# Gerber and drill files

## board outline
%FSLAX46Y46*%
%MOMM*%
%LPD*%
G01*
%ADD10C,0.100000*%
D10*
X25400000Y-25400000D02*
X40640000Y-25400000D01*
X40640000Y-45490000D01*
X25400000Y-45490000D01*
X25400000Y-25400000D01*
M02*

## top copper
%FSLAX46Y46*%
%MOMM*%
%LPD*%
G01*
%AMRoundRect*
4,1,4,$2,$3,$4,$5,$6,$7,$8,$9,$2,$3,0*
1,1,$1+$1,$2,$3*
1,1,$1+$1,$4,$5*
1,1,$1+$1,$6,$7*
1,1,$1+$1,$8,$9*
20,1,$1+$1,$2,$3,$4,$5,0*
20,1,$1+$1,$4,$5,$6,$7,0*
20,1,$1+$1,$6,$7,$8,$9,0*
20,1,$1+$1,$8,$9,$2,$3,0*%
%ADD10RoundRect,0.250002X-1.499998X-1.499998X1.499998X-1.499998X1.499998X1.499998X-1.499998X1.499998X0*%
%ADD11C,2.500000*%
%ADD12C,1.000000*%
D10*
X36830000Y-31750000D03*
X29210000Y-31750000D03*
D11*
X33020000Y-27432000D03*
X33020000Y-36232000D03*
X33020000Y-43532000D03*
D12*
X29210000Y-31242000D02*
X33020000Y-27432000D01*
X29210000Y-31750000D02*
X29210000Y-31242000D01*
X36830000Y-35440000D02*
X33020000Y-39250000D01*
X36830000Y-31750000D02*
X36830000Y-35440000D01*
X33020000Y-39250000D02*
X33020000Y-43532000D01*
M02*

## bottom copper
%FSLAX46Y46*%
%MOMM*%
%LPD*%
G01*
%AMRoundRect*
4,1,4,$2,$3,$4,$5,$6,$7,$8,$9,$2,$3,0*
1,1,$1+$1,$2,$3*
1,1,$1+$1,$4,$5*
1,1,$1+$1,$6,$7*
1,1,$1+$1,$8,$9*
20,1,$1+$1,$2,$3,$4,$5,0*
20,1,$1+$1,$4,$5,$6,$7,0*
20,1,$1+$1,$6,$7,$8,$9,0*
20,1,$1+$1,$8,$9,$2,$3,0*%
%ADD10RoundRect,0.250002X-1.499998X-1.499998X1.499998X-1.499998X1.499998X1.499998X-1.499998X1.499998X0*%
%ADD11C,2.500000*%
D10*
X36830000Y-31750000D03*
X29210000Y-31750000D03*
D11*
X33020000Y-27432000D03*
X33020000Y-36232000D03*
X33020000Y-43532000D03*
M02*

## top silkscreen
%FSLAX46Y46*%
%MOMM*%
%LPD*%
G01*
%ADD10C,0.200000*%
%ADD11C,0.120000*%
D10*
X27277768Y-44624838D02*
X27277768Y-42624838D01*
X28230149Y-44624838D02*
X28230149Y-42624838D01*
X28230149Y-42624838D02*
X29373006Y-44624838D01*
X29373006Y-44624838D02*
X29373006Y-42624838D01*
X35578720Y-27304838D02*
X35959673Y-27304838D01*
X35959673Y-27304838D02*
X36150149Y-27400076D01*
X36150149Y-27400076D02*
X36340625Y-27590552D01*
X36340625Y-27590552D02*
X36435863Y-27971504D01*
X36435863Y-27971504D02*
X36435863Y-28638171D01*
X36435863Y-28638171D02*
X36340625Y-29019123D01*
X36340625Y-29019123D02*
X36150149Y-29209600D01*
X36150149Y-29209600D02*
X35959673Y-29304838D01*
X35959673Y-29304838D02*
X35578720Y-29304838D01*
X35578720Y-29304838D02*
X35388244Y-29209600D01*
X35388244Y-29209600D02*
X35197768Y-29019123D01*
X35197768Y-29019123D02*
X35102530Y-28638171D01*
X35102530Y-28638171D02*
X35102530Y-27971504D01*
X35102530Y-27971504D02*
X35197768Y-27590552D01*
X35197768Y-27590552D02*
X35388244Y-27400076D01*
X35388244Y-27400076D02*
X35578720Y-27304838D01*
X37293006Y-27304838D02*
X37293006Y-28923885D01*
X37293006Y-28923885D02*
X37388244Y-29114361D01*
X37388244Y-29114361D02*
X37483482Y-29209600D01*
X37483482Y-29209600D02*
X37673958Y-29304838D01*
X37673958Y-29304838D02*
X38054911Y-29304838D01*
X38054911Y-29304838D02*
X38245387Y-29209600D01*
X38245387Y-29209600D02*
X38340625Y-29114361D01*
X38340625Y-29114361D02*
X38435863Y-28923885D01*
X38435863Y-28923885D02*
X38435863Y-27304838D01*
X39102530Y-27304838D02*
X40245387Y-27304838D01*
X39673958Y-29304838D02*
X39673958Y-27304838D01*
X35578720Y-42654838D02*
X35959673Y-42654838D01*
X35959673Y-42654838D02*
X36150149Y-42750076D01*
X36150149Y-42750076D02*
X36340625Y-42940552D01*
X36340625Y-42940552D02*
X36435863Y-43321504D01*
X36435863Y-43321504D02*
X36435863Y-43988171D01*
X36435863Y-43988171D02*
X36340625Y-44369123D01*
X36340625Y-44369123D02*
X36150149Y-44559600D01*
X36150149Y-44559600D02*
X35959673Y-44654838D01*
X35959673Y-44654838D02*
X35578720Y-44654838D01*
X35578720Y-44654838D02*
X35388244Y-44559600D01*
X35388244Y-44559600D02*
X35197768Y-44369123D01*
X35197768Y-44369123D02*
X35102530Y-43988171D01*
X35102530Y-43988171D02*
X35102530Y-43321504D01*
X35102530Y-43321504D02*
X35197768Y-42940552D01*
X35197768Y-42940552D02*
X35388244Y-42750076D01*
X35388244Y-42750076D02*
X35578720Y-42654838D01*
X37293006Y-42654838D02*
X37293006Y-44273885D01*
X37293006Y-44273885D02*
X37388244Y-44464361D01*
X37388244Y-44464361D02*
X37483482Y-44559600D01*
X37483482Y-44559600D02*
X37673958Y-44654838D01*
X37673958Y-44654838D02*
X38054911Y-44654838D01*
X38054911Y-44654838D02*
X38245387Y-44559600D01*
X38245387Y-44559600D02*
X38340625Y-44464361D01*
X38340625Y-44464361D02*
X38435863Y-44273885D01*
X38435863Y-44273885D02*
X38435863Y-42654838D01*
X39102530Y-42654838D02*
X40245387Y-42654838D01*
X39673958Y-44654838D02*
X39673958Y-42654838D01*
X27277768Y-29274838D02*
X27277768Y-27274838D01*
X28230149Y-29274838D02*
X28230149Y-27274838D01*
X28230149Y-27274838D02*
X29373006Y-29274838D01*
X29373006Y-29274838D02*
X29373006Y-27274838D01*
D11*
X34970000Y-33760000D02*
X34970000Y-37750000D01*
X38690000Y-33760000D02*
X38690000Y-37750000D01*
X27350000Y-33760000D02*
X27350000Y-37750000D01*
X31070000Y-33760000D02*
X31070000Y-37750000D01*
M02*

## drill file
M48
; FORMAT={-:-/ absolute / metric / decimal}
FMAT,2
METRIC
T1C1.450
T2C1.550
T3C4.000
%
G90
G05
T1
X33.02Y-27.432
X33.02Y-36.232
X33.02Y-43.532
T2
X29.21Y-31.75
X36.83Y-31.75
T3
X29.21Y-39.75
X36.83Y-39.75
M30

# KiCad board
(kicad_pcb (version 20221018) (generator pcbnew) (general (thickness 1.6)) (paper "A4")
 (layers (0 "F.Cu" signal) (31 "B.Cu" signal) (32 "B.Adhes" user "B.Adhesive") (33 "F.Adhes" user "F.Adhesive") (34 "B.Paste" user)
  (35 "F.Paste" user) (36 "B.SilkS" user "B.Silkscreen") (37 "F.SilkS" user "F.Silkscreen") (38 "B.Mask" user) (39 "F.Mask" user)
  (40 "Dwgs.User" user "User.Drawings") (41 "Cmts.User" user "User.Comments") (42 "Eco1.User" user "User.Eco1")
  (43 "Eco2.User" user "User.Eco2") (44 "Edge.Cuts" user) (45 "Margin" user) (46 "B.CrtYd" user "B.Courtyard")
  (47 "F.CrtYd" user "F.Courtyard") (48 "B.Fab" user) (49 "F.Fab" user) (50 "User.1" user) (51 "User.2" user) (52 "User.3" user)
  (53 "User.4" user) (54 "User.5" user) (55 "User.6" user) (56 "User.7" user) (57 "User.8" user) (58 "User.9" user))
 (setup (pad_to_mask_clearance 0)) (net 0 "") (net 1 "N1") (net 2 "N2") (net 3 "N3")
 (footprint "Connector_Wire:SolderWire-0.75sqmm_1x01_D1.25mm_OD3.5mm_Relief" (layer "F.Cu") (at 36.83 31.75)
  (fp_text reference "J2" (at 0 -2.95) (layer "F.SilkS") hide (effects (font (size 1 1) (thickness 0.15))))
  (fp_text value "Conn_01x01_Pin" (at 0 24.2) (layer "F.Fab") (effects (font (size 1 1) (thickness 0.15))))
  (fp_line (start -1.86 2.01) (end -1.86 6) (stroke (width 0.12) (type solid)) (layer "F.SilkS"))
  (fp_line (start 1.86 2.01) (end 1.86 6) (stroke (width 0.12) (type solid)) (layer "F.SilkS"))
  (pad "" np_thru_hole circle (at 0 8) (size 4 4) (drill 4) (layers "*.Cu" "*.Mask"))
  (pad "1" thru_hole roundrect (at 0 0) (size 3.5 3.5) (drill 1.55) (layers "*.Cu" "*.Mask") (roundrect_rratio 0.071429) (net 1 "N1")))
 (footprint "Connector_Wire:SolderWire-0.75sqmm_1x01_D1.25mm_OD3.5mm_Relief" (layer "F.Cu") (at 29.21 31.75)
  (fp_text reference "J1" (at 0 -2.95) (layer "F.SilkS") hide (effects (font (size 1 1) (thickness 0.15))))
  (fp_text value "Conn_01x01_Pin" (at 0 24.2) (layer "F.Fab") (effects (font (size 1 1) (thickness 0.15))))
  (fp_line (start -1.86 2.01) (end -1.86 6) (stroke (width 0.12) (type solid)) (layer "F.SilkS"))
  (fp_line (start 1.86 2.01) (end 1.86 6) (stroke (width 0.12) (type solid)) (layer "F.SilkS"))
  (pad "" np_thru_hole circle (at 0 8) (size 4 4) (drill 4) (layers "*.Cu" "*.Mask"))
  (pad "1" thru_hole roundrect (at 0 0) (size 3.5 3.5) (drill 1.55) (layers "*.Cu" "*.Mask") (roundrect_rratio 0.071429) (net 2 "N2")))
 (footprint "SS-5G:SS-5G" (layer "F.Cu") (at 33.02 27.432)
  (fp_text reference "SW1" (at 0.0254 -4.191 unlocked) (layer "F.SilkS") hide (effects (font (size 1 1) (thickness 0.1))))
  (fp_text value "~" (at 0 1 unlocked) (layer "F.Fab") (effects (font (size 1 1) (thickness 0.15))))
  (pad "1" thru_hole circle (at 0 0) (size 2.5 2.5) (drill 1.45) (layers "*.Cu" "*.Mask") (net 2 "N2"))
  (pad "2" thru_hole circle (at 0 8.8) (size 2.5 2.5) (drill 1.45) (layers "*.Cu" "*.Mask") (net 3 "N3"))
  (pad "3" thru_hole circle (at 0 16.1) (size 2.5 2.5) (drill 1.45) (layers "*.Cu" "*.Mask") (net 1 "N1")))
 (gr_rect (start 25.4 25.4) (end 40.64 45.49) (stroke (width 0.1) (type default)) (fill none) (layer "Edge.Cuts"))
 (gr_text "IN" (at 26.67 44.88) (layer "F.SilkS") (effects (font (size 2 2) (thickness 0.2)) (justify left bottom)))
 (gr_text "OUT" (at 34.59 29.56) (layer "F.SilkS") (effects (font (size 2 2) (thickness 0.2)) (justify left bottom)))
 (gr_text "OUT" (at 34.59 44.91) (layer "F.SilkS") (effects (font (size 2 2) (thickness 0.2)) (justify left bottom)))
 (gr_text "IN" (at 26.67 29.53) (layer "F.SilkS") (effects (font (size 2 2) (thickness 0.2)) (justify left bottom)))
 (segment (start 29.21 31.242) (end 33.02 27.432) (width 1) (layer "F.Cu") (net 2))
 (segment (start 29.21 31.75) (end 29.21 31.242) (width 1) (layer "F.Cu") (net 2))
 (segment (start 36.83 35.44) (end 33.02 39.25) (width 1) (layer "F.Cu") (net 1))
 (segment (start 36.83 31.75) (end 36.83 35.44) (width 1) (layer "F.Cu") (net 1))
 (segment (start 33.02 39.25) (end 33.02 43.532) (width 1) (layer "F.Cu") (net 1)))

